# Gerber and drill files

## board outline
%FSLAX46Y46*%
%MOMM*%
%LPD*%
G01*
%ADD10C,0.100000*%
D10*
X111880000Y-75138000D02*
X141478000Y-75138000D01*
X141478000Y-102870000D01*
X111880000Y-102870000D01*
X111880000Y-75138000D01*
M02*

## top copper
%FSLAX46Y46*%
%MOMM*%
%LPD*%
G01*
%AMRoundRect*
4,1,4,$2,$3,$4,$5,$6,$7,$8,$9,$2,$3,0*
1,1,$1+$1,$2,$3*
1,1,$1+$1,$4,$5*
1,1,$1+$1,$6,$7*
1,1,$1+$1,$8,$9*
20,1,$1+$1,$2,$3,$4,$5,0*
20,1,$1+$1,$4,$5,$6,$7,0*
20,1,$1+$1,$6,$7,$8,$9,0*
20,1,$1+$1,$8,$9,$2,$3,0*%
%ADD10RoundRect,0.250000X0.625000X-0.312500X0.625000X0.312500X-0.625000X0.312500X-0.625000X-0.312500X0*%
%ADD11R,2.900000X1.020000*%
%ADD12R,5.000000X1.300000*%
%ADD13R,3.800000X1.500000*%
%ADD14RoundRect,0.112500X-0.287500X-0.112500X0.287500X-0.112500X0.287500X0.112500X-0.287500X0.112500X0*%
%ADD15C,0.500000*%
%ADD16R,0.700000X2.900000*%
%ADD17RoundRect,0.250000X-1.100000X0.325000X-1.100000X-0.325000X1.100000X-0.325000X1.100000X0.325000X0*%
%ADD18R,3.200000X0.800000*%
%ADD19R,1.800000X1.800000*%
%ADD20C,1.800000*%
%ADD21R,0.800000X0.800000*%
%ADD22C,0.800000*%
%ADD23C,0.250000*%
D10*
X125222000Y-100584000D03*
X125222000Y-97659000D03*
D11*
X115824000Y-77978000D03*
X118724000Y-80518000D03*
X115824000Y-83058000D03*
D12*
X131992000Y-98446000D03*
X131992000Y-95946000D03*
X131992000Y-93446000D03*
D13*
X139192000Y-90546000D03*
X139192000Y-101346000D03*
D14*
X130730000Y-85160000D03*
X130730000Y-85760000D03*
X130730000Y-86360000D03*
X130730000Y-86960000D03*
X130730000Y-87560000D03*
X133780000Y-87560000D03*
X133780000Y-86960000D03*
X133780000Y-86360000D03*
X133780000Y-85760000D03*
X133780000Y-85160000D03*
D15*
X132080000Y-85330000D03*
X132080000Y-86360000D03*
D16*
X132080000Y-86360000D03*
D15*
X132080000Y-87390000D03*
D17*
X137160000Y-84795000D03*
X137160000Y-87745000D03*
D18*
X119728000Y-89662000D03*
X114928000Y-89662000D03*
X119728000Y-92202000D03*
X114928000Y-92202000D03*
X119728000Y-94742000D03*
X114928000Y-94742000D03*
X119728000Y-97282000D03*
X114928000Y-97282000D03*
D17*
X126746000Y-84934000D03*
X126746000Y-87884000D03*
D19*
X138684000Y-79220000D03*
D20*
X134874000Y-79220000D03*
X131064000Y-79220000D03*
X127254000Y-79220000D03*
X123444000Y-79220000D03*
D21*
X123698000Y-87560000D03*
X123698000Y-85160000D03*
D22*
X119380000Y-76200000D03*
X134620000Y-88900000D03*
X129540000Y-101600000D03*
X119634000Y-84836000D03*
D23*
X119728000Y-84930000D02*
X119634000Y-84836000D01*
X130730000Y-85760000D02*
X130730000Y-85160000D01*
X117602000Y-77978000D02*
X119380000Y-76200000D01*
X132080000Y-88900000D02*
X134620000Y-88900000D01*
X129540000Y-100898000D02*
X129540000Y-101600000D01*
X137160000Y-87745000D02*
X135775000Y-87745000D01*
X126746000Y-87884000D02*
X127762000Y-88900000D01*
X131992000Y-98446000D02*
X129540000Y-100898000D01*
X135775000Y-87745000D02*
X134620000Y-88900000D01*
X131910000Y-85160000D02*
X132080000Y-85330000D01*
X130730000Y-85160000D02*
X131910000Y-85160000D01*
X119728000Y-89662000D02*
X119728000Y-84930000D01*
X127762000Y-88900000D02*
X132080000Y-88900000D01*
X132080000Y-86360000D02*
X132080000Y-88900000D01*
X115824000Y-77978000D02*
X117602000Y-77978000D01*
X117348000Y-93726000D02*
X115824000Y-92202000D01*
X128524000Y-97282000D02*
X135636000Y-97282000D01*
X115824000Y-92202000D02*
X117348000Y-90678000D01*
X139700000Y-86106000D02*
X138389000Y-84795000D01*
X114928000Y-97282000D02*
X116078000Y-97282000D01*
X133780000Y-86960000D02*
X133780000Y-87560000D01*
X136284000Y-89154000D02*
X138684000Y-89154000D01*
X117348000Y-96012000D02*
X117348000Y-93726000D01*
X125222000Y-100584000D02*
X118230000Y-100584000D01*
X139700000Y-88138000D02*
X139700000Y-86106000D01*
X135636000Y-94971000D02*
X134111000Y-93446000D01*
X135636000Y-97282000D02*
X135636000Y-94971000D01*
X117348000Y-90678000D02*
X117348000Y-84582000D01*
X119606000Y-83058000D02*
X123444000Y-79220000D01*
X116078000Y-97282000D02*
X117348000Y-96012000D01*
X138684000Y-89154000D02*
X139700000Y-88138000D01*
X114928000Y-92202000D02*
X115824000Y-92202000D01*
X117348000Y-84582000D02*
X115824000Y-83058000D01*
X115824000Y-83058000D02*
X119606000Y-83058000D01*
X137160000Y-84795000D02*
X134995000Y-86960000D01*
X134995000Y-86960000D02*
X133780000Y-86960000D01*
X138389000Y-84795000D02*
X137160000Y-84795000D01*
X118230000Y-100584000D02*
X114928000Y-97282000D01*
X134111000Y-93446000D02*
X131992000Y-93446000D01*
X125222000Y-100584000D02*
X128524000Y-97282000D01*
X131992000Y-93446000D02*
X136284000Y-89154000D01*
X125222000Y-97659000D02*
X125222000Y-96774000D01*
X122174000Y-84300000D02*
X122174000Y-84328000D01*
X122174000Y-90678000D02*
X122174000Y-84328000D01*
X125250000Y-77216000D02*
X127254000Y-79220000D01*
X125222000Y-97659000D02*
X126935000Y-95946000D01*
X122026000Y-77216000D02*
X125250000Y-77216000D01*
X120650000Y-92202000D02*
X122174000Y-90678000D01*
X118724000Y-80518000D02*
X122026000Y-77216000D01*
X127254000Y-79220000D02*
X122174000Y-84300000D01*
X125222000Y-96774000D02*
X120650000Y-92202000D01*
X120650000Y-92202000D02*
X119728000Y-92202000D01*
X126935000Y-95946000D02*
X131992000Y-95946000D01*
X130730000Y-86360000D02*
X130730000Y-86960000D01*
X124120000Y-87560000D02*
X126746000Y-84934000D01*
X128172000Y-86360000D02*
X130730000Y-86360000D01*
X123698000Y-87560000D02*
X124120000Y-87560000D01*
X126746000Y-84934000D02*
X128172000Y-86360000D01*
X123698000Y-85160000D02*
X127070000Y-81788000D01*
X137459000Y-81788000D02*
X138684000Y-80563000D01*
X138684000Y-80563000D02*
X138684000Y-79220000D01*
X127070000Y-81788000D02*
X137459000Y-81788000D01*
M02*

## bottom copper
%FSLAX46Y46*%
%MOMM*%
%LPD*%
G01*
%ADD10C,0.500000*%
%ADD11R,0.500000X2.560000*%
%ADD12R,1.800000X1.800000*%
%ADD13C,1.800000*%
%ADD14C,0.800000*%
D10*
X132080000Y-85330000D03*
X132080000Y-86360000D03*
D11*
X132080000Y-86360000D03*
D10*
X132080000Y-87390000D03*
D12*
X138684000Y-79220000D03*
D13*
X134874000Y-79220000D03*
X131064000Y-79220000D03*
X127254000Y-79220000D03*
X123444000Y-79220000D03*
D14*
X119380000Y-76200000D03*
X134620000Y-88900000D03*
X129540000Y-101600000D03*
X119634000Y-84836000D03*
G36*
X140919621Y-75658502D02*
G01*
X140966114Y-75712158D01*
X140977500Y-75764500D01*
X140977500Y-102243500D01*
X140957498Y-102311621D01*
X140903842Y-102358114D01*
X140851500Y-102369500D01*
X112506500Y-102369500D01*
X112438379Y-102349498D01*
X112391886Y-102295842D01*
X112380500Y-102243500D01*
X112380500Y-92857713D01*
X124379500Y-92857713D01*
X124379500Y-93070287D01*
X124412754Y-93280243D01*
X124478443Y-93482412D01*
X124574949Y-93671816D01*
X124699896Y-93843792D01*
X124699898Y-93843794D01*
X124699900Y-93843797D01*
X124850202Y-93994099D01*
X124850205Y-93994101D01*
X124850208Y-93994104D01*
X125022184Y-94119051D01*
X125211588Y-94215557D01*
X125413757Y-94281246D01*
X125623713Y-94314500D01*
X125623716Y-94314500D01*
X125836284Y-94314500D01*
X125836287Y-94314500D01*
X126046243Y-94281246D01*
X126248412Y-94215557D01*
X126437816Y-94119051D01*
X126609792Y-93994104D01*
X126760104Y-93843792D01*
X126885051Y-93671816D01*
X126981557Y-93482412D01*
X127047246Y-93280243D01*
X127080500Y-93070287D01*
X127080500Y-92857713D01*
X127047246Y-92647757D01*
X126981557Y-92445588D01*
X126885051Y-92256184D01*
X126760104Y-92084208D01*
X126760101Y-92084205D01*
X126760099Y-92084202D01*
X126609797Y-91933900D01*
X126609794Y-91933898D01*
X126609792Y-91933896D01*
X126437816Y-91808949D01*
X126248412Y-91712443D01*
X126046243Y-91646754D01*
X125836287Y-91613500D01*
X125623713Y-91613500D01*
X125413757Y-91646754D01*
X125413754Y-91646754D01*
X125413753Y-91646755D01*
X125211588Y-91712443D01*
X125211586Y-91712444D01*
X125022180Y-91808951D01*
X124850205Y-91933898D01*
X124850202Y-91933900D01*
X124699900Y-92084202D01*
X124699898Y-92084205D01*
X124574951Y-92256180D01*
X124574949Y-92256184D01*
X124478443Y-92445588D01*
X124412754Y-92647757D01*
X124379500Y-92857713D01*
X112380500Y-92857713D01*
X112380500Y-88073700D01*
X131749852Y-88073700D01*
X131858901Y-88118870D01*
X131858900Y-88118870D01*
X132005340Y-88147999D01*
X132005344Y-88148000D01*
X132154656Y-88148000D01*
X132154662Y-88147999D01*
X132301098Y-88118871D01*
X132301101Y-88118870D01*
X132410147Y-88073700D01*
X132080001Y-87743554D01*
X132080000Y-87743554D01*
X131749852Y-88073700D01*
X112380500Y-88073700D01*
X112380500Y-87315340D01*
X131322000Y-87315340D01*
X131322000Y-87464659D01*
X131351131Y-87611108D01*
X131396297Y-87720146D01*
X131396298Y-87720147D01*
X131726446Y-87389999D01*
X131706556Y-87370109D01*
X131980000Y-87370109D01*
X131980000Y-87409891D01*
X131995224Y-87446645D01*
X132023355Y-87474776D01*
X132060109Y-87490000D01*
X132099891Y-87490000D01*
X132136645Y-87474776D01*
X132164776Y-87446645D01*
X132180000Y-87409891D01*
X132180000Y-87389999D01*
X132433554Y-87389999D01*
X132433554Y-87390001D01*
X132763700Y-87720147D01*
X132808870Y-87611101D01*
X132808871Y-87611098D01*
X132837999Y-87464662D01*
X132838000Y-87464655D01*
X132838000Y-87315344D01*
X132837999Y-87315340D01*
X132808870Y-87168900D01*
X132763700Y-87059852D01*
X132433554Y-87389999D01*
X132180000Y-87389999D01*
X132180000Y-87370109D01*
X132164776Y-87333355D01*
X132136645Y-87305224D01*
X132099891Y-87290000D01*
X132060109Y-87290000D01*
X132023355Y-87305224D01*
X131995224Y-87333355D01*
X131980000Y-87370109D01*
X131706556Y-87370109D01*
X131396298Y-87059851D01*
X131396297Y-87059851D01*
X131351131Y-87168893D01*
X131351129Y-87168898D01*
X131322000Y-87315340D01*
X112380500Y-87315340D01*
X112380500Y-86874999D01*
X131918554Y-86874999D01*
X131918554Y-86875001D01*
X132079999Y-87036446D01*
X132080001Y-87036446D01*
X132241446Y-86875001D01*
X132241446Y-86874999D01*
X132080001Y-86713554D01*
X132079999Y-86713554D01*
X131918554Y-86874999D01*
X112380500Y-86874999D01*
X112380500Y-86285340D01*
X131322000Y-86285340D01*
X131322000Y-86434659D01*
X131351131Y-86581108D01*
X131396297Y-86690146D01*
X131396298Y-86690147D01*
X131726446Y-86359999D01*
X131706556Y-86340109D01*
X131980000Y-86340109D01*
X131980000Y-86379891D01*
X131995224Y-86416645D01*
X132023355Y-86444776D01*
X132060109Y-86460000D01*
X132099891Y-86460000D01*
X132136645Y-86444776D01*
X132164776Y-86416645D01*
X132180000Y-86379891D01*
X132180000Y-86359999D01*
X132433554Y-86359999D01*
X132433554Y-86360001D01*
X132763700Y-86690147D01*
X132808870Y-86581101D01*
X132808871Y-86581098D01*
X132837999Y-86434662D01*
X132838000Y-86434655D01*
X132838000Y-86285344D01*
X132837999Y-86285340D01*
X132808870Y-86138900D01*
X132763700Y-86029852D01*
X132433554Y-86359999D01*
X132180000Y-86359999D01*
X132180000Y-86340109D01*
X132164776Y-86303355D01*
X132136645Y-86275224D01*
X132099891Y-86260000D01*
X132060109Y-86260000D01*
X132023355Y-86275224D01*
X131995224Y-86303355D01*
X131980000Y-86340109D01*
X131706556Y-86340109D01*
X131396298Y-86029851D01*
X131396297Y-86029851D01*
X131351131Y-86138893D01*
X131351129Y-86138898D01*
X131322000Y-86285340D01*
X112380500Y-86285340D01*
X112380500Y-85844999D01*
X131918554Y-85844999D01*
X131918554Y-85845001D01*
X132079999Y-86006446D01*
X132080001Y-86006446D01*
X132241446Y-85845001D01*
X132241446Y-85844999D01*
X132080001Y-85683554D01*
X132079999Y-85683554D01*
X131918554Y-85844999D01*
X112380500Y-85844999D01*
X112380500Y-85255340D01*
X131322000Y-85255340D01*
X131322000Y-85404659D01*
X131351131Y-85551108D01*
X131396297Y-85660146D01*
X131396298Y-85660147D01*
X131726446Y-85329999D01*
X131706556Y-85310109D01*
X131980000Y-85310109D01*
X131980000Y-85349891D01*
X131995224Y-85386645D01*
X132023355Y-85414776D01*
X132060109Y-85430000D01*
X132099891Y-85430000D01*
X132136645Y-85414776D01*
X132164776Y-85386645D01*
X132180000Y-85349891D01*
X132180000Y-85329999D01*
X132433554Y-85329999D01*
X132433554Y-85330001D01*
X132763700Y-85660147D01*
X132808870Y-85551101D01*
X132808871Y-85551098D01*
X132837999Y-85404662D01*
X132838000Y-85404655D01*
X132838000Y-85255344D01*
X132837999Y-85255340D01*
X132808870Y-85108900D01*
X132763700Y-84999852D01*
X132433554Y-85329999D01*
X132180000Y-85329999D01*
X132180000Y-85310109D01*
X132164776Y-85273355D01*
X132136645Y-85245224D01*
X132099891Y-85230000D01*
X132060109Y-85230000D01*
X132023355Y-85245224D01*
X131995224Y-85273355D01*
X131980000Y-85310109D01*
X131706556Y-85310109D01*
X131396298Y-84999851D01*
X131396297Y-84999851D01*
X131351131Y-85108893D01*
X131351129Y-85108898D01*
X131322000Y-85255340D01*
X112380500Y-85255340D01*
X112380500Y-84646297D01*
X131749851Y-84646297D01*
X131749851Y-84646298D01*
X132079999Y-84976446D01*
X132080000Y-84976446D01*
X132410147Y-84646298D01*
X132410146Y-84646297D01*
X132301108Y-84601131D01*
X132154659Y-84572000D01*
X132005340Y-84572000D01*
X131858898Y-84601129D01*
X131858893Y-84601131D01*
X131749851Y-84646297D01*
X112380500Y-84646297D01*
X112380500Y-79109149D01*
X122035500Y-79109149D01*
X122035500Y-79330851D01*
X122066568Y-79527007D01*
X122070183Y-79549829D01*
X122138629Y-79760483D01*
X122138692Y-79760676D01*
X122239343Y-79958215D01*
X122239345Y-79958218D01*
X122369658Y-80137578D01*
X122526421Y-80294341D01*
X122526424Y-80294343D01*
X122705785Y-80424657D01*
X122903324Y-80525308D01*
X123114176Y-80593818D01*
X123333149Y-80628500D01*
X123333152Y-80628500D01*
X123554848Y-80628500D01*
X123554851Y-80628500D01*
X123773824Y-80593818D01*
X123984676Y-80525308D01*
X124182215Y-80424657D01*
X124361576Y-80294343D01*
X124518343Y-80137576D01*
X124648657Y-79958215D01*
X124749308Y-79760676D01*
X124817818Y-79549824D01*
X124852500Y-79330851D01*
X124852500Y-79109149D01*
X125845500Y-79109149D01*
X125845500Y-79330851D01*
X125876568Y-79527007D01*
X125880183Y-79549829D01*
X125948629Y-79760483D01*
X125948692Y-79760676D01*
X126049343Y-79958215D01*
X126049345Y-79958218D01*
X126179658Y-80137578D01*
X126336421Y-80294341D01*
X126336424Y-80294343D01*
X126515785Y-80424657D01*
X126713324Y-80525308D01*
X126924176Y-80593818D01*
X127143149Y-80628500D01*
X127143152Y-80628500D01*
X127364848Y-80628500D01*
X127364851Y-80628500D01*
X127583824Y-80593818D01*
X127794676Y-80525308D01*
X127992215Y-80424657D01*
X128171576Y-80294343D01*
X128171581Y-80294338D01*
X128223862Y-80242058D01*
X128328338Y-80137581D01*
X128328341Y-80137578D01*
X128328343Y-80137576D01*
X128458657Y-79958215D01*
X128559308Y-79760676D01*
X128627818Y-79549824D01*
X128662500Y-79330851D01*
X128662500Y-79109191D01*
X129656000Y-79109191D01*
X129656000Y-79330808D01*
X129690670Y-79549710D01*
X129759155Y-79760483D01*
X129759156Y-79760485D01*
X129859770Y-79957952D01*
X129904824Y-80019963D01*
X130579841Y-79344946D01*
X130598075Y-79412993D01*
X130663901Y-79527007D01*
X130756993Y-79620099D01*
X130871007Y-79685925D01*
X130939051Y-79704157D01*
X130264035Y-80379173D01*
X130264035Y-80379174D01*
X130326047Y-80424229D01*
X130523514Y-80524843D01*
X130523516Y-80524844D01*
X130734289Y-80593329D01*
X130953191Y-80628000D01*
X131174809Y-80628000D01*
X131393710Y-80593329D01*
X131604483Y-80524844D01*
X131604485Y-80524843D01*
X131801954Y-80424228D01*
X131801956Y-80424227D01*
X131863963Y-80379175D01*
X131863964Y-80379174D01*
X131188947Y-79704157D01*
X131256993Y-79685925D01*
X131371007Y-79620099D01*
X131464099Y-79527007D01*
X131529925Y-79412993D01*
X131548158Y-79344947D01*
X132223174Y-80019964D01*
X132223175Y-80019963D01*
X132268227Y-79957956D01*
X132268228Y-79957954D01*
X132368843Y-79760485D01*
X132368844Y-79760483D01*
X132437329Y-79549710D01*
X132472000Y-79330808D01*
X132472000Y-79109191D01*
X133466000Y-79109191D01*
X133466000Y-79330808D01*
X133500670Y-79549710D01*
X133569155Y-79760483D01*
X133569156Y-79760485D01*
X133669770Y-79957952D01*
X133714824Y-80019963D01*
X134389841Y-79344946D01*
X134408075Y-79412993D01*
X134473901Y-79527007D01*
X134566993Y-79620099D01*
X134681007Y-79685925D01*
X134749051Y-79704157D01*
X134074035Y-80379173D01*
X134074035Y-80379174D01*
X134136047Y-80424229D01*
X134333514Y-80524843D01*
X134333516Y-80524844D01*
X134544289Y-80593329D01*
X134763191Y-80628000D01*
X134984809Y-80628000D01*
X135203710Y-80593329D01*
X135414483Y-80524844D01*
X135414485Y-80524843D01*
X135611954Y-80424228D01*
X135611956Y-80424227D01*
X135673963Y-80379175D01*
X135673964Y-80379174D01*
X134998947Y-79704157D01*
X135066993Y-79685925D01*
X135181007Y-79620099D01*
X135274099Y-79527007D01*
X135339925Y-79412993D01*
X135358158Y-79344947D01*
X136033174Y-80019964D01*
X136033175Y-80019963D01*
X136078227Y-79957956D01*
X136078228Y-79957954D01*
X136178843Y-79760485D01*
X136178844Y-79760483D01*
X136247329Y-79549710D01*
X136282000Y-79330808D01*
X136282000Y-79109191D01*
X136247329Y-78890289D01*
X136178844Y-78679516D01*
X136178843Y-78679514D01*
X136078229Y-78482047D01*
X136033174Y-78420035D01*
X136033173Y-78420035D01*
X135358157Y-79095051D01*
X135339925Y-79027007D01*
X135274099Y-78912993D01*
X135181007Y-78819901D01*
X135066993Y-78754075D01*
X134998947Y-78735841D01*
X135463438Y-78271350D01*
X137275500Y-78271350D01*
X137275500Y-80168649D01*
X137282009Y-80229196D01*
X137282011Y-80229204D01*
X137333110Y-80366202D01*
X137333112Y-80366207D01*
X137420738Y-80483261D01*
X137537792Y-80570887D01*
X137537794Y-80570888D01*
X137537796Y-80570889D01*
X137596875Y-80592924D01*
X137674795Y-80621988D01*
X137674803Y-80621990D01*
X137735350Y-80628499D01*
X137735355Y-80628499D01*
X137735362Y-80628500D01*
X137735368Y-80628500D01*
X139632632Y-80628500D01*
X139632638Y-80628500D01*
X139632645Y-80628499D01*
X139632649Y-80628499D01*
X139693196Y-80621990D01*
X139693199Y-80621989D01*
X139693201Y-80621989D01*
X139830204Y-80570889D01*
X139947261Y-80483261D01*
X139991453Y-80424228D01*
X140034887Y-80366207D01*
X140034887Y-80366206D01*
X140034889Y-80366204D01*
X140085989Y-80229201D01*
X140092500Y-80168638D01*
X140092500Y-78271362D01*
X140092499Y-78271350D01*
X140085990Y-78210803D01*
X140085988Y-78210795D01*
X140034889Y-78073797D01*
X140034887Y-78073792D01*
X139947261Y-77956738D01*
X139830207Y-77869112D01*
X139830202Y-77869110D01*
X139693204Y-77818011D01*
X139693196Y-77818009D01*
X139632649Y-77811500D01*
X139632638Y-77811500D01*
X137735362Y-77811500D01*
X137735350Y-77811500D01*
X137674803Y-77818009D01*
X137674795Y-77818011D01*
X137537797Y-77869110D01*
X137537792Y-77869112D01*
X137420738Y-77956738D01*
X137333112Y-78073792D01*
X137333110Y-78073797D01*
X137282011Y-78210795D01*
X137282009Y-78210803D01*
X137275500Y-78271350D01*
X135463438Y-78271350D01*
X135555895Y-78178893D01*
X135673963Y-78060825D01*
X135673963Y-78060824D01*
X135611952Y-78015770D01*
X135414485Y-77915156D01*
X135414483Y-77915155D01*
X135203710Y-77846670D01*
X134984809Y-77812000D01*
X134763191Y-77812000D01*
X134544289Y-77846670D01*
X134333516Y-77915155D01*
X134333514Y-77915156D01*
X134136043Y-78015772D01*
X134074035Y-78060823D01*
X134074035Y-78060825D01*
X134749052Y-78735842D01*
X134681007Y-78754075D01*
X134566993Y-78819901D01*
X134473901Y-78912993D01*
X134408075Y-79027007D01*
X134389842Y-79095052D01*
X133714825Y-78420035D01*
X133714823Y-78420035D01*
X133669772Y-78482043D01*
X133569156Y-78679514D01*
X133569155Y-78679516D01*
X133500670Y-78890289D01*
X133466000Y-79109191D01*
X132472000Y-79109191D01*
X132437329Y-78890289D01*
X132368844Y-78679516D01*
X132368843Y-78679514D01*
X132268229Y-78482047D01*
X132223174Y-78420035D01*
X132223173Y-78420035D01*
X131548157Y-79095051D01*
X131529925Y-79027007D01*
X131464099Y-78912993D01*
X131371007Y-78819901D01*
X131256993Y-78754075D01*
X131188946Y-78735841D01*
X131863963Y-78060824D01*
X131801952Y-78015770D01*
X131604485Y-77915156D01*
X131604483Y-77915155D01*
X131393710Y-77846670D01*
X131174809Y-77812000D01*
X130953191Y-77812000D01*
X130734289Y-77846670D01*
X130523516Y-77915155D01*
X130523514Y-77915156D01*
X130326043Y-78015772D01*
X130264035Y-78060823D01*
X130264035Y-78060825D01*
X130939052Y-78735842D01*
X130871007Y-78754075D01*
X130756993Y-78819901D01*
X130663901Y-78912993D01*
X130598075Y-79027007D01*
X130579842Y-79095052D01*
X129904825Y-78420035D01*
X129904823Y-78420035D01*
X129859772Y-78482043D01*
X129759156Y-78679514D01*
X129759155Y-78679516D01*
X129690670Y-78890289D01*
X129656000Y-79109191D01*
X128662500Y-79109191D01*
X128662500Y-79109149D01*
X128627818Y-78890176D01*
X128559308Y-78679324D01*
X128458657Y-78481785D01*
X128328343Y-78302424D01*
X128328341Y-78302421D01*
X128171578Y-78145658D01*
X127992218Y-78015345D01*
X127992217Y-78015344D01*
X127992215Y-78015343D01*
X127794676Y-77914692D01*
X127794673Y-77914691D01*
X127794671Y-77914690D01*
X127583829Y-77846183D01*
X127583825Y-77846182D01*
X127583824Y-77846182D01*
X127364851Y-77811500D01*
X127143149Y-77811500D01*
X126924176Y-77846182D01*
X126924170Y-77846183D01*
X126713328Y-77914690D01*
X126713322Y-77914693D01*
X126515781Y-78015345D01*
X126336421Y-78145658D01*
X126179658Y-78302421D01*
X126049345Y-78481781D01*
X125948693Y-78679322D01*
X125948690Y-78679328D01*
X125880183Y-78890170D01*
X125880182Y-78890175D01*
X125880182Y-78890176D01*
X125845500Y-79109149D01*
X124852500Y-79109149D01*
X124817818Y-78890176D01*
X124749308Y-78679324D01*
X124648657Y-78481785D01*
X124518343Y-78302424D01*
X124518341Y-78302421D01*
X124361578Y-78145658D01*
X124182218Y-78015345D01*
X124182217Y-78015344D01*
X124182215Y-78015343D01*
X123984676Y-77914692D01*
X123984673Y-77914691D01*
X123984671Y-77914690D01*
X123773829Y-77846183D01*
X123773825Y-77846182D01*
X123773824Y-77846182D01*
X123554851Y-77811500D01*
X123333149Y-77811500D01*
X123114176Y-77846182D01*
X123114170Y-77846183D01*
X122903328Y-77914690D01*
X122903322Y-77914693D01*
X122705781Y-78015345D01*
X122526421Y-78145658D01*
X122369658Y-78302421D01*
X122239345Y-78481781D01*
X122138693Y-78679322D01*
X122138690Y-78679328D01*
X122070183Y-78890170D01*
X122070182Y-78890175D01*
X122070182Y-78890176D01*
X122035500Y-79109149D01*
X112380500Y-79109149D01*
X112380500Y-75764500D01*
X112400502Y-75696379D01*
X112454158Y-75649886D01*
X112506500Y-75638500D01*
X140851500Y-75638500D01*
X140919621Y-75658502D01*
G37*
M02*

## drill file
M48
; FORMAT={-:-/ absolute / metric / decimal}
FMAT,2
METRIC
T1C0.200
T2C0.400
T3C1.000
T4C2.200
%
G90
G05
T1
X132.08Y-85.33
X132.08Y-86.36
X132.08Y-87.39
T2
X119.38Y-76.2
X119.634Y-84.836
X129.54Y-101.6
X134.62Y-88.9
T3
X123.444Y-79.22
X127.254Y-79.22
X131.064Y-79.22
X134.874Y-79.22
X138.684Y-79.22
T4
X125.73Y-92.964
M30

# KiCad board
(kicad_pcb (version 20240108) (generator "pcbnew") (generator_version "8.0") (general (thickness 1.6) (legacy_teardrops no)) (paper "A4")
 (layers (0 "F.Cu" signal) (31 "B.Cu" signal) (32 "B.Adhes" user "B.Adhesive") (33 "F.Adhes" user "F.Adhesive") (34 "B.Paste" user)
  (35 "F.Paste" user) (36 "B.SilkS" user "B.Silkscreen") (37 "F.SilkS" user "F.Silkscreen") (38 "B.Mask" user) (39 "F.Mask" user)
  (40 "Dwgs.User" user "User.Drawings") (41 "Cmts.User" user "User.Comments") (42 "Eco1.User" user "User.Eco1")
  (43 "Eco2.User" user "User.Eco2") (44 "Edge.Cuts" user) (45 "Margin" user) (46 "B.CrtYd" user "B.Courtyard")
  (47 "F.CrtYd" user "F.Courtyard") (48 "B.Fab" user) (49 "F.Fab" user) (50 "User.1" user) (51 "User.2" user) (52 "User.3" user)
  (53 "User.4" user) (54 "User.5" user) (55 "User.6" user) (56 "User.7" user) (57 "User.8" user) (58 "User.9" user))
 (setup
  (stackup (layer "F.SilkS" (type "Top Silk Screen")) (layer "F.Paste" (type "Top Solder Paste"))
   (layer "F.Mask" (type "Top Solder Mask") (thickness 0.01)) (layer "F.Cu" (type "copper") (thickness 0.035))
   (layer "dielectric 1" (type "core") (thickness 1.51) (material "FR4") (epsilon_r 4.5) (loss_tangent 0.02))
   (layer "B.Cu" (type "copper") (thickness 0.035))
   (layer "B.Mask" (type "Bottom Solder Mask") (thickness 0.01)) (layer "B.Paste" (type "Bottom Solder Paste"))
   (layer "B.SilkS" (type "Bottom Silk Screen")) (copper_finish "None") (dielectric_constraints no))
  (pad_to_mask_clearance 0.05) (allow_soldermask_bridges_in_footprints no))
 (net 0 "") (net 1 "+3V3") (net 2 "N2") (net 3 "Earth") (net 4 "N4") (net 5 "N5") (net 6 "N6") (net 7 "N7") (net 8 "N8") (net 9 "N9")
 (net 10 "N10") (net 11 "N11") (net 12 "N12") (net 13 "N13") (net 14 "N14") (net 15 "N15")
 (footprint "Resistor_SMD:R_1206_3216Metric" (layer "F.Cu") (at 125.222 99.1215 90)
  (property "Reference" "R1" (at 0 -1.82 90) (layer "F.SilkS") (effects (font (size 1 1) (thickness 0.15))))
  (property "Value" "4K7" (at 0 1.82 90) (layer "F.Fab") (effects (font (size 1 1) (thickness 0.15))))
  (pad "1" smd roundrect (at -1.4625 0 90) (size 1.125 1.75) (layers "F.Cu" "F.Paste" "F.Mask") (roundrect_rratio 0.222222) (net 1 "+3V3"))
  (pad "2" smd roundrect (at 1.4625 0 90) (size 1.125 1.75) (layers "F.Cu" "F.Paste" "F.Mask") (roundrect_rratio 0.222222) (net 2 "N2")))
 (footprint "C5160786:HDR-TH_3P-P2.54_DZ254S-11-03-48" (layer "F.Cu") (at 117.274 80.518 -90)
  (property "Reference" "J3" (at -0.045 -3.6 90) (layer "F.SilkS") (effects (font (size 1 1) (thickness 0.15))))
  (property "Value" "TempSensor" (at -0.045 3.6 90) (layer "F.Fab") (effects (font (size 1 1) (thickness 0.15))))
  (pad "1" smd rect (at -2.54 1.45 270) (size 1.02 2.9) (layers "F.Cu" "F.Paste" "F.Mask") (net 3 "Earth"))
  (pad "2" smd rect (at 0 -1.45 270) (size 1.02 2.9) (layers "F.Cu" "F.Paste" "F.Mask") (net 2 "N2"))
  (pad "3" smd rect (at 2.54 1.45 270) (size 1.02 2.9) (layers "F.Cu" "F.Paste" "F.Mask") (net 1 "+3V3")))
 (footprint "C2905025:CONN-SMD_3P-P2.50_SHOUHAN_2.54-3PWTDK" (layer "F.Cu") (at 135.592 95.946 90)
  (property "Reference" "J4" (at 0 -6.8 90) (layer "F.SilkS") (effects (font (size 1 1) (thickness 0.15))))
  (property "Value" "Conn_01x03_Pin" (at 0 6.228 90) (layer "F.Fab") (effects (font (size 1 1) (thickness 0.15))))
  (pad "1" smd rect (at -2.5 -3.6 90) (size 1.3 5) (layers "F.Cu" "F.Paste" "F.Mask") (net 3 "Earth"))
  (pad "2" smd rect (at 0 -3.6 90) (size 1.3 5) (layers "F.Cu" "F.Paste" "F.Mask") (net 2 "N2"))
  (pad "3" smd rect (at 2.5 -3.6 90) (size 1.3 5) (layers "F.Cu" "F.Paste" "F.Mask") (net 1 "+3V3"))
  (pad "4" smd rect (at 5.4 3.6 90) (size 1.5 3.8) (layers "F.Cu" "F.Paste" "F.Mask") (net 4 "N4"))
  (pad "5" smd rect (at -5.4 3.6 90) (size 1.5 3.8) (layers "F.Cu" "F.Paste" "F.Mask") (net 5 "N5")))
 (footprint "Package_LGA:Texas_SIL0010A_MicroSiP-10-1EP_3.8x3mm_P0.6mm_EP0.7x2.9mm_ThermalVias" (layer "F.Cu") (at 132.255 86.36)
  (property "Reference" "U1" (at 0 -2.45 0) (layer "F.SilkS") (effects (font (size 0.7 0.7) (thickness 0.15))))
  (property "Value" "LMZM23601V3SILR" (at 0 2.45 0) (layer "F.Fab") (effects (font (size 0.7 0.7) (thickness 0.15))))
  (pad "" smd roundrect (at -0.175 -0.97) (size 0.65 0.9) (layers "F.Paste") (roundrect_rratio 0.25))
  (pad "" smd roundrect (at -0.175 0) (size 0.65 0.9) (layers "F.Paste") (roundrect_rratio 0.25))
  (pad "" smd roundrect (at -0.175 0.97) (size 0.65 0.9) (layers "F.Paste") (roundrect_rratio 0.25))
  (pad "1" smd roundrect (at -1.525 -1.2) (size 0.8 0.45) (layers "F.Cu" "F.Paste" "F.Mask") (roundrect_rratio 0.25) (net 3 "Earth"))
  (pad "2" smd roundrect (at -1.525 -0.6) (size 0.8 0.45) (layers "F.Cu" "F.Paste" "F.Mask") (roundrect_rratio 0.25) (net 3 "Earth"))
  (pad "3" smd roundrect (at -1.525 0) (size 0.8 0.45) (layers "F.Cu" "F.Paste" "F.Mask") (roundrect_rratio 0.25) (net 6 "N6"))
  (pad "4" smd roundrect (at -1.525 0.6) (size 0.8 0.45) (layers "F.Cu" "F.Paste" "F.Mask") (roundrect_rratio 0.25) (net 6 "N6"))
  (pad "5" smd roundrect (at -1.525 1.2) (size 0.8 0.45) (layers "F.Cu" "F.Paste" "F.Mask") (roundrect_rratio 0.25) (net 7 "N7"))
  (pad "6" smd roundrect (at 1.525 1.2) (size 0.8 0.45) (layers "F.Cu" "F.Paste" "F.Mask") (roundrect_rratio 0.25) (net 1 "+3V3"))
  (pad "7" smd roundrect (at 1.525 0.6) (size 0.8 0.45) (layers "F.Cu" "F.Paste" "F.Mask") (roundrect_rratio 0.25) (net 1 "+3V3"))
  (pad "8" smd roundrect (at 1.525 0) (size 0.8 0.45) (layers "F.Cu" "F.Paste" "F.Mask") (roundrect_rratio 0.25) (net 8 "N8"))
  (pad "9" smd roundrect (at 1.525 -0.6) (size 0.8 0.45) (layers "F.Cu" "F.Paste" "F.Mask") (roundrect_rratio 0.25) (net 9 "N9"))
  (pad "10" smd roundrect (at 1.525 -1.2) (size 0.8 0.45) (layers "F.Cu" "F.Paste" "F.Mask") (roundrect_rratio 0.25) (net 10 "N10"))
  (pad "11" thru_hole circle (at -0.175 -1.03) (size 0.5 0.5) (drill 0.2) (layers "*.Cu") (remove_unused_layers no) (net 3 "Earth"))
  (pad "11" thru_hole circle (at -0.175 0) (size 0.5 0.5) (drill 0.2) (layers "*.Cu") (remove_unused_layers no) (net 3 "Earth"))
  (pad "11" smd rect (at -0.175 0) (size 0.5 2.56) (layers "B.Cu") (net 3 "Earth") (zone_connect 2))
  (pad "11" smd rect (at -0.175 0) (size 0.7 2.9) (layers "F.Cu" "F.Mask") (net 3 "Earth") (zone_connect 2))
  (pad "11" thru_hole circle (at -0.175 1.03) (size 0.5 0.5) (drill 0.2) (layers "*.Cu") (remove_unused_layers no) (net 3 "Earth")))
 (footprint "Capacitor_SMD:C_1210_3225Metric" (layer "F.Cu") (at 137.16 86.27 -90)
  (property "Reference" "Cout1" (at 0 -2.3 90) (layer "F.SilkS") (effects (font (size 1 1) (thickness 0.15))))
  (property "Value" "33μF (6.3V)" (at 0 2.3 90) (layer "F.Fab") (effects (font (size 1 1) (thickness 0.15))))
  (pad "1" smd roundrect (at -1.475 0 270) (size 1.15 2.7) (layers "F.Cu" "F.Paste" "F.Mask") (roundrect_rratio 0.217391) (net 1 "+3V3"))
  (pad "2" smd roundrect (at 1.475 0 270) (size 1.15 2.7) (layers "F.Cu" "F.Paste" "F.Mask") (roundrect_rratio 0.217391) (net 3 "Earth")))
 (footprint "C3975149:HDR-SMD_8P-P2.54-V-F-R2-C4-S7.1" (layer "F.Cu") (at 117.328 93.472 -90)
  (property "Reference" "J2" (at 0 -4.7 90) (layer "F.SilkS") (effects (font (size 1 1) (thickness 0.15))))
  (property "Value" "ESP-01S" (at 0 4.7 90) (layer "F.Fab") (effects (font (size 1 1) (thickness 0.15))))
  (pad "1" smd rect (at -3.81 -2.4 270) (size 0.8 3.2) (layers "F.Cu" "F.Paste" "F.Mask") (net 3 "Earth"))
  (pad "2" smd rect (at -3.81 2.4 270) (size 0.8 3.2) (layers "F.Cu" "F.Paste" "F.Mask") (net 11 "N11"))
  (pad "3" smd rect (at -1.27 -2.4 270) (size 0.8 3.2) (layers "F.Cu" "F.Paste" "F.Mask") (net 2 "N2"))
  (pad "4" smd rect (at -1.27 2.4 270) (size 0.8 3.2) (layers "F.Cu" "F.Paste" "F.Mask") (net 1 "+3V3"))
  (pad "5" smd rect (at 1.27 -2.4 270) (size 0.8 3.2) (layers "F.Cu" "F.Paste" "F.Mask") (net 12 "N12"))
  (pad "6" smd rect (at 1.27 2.4 270) (size 0.8 3.2) (layers "F.Cu" "F.Paste" "F.Mask") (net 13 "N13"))
  (pad "7" smd rect (at 3.81 -2.4 270) (size 0.8 3.2) (layers "F.Cu" "F.Paste" "F.Mask") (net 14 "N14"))
  (pad "8" smd rect (at 3.81 2.4 270) (size 0.8 3.2) (layers "F.Cu" "F.Paste" "F.Mask") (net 1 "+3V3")))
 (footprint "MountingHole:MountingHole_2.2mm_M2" (layer "F.Cu") (at 125.73 92.964)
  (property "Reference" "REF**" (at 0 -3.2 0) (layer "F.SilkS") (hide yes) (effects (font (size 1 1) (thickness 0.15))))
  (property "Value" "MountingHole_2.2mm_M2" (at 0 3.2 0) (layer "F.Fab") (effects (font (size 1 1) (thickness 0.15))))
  (pad "" np_thru_hole circle (at 0 0) (size 2.2 2.2) (drill 2.2) (layers "*.Cu" "*.Mask")))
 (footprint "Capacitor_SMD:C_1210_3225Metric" (layer "F.Cu") (at 126.746 86.409 -90)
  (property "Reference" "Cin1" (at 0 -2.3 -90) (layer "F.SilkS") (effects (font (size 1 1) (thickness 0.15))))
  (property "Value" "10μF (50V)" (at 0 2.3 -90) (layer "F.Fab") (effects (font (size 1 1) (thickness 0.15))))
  (pad "1" smd roundrect (at -1.475 0 270) (size 1.15 2.7) (layers "F.Cu" "F.Paste" "F.Mask") (roundrect_rratio 0.217391) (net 6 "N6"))
  (pad "2" smd roundrect (at 1.475 0 270) (size 1.15 2.7) (layers "F.Cu" "F.Paste" "F.Mask") (roundrect_rratio 0.217391) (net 3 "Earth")))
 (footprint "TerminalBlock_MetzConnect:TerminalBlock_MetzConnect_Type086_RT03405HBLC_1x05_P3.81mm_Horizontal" (layer "F.Cu")
  (at 138.684 79.22 180)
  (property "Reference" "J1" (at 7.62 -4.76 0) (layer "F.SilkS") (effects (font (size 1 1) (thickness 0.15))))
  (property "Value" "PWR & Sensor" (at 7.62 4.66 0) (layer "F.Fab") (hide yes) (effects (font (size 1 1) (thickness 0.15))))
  (pad "1" thru_hole rect (at 0 0 180) (size 1.8 1.8) (drill 1) (layers "*.Cu" "*.Mask") (remove_unused_layers no) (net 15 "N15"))
  (pad "2" thru_hole circle (at 3.81 0 180) (size 1.8 1.8) (drill 1) (layers "*.Cu" "*.Mask") (remove_unused_layers no) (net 3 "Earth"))
  (pad "3" thru_hole circle (at 7.62 0 180) (size 1.8 1.8) (drill 1) (layers "*.Cu" "*.Mask") (remove_unused_layers no) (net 3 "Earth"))
  (pad "4" thru_hole circle (at 11.43 0 180) (size 1.8 1.8) (drill 1) (layers "*.Cu" "*.Mask") (remove_unused_layers no) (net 2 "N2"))
  (pad "5" thru_hole circle (at 15.24 0 180) (size 1.8 1.8) (drill 1) (layers "*.Cu" "*.Mask") (remove_unused_layers no) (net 1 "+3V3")))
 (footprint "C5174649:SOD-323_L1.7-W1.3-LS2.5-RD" (layer "F.Cu") (at 123.698 86.36 90)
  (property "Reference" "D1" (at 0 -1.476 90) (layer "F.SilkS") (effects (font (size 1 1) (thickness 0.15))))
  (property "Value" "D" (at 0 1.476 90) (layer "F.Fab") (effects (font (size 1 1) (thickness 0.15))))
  (pad "1" smd rect (at -1.2 0 90) (size 0.8 0.8) (layers "F.Cu" "F.Paste" "F.Mask") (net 6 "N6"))
  (pad "2" smd rect (at 1.2 0 90) (size 0.8 0.8) (layers "F.Cu" "F.Paste" "F.Mask") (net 15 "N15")))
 (gr_rect (start 111.88 75.138) (end 141.478 102.87) (stroke (width 0.1) (type solid)) (fill none) (layer "Edge.Cuts"))
 (segment (start 119.728 84.93) (end 119.634 84.836) (width 0.25) (layer "F.Cu") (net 3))
 (segment (start 130.73 85.76) (end 130.73 85.16) (width 0.25) (layer "F.Cu") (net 3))
 (segment (start 117.602 77.978) (end 119.38 76.2) (width 0.25) (layer "F.Cu") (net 3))
 (segment (start 132.08 88.9) (end 134.62 88.9) (width 0.25) (layer "F.Cu") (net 3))
 (segment (start 129.54 100.898) (end 129.54 101.6) (width 0.25) (layer "F.Cu") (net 3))
 (segment (start 137.16 87.745) (end 135.775 87.745) (width 0.25) (layer "F.Cu") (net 3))
 (segment (start 126.746 87.884) (end 127.762 88.9) (width 0.25) (layer "F.Cu") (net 3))
 (segment (start 131.992 98.446) (end 129.54 100.898) (width 0.25) (layer "F.Cu") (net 3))
 (segment (start 135.775 87.745) (end 134.62 88.9) (width 0.25) (layer "F.Cu") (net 3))
 (segment (start 131.91 85.16) (end 132.08 85.33) (width 0.25) (layer "F.Cu") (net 3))
 (segment (start 130.73 85.16) (end 131.91 85.16) (width 0.25) (layer "F.Cu") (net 3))
 (segment (start 119.728 89.662) (end 119.728 84.93) (width 0.25) (layer "F.Cu") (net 3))
 (segment (start 127.762 88.9) (end 132.08 88.9) (width 0.25) (layer "F.Cu") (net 3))
 (segment (start 132.08 86.36) (end 132.08 88.9) (width 0.25) (layer "F.Cu") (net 3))
 (segment (start 115.824 77.978) (end 117.602 77.978) (width 0.25) (layer "F.Cu") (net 3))
 (via (at 119.38 76.2) (size 0.8) (drill 0.4) (layers "F.Cu" "B.Cu") (free yes) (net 3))
 (via (at 134.62 88.9) (size 0.8) (drill 0.4) (layers "F.Cu" "B.Cu") (free yes) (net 3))
 (via (at 129.54 101.6) (size 0.8) (drill 0.4) (layers "F.Cu" "B.Cu") (free yes) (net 3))
 (via (at 119.634 84.836) (size 0.8) (drill 0.4) (layers "F.Cu" "B.Cu") (free yes) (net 3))
 (segment (start 117.348 93.726) (end 115.824 92.202) (width 0.25) (layer "F.Cu") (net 1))
 (segment (start 128.524 97.282) (end 135.636 97.282) (width 0.25) (layer "F.Cu") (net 1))
 (segment (start 115.824 92.202) (end 117.348 90.678) (width 0.25) (layer "F.Cu") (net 1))
 (segment (start 139.7 86.106) (end 138.389 84.795) (width 0.25) (layer "F.Cu") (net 1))
 (segment (start 114.928 97.282) (end 116.078 97.282) (width 0.25) (layer "F.Cu") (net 1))
 (segment (start 133.78 86.96) (end 133.78 87.56) (width 0.25) (layer "F.Cu") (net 1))
 (segment (start 136.284 89.154) (end 138.684 89.154) (width 0.25) (layer "F.Cu") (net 1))
 (segment (start 117.348 96.012) (end 117.348 93.726) (width 0.25) (layer "F.Cu") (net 1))
 (segment (start 125.222 100.584) (end 118.23 100.584) (width 0.25) (layer "F.Cu") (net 1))
 (segment (start 139.7 88.138) (end 139.7 86.106) (width 0.25) (layer "F.Cu") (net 1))
 (segment (start 135.636 94.971) (end 134.111 93.446) (width 0.25) (layer "F.Cu") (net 1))
 (segment (start 135.636 97.282) (end 135.636 94.971) (width 0.25) (layer "F.Cu") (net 1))
 (segment (start 117.348 90.678) (end 117.348 84.582) (width 0.25) (layer "F.Cu") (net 1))
 (segment (start 119.606 83.058) (end 123.444 79.22) (width 0.25) (layer "F.Cu") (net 1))
 (segment (start 116.078 97.282) (end 117.348 96.012) (width 0.25) (layer "F.Cu") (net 1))
 (segment (start 138.684 89.154) (end 139.7 88.138) (width 0.25) (layer "F.Cu") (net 1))
 (segment (start 114.928 92.202) (end 115.824 92.202) (width 0.25) (layer "F.Cu") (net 1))
 (segment (start 117.348 84.582) (end 115.824 83.058) (width 0.25) (layer "F.Cu") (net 1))
 (segment (start 115.824 83.058) (end 119.606 83.058) (width 0.25) (layer "F.Cu") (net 1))
 (segment (start 137.16 84.795) (end 134.995 86.96) (width 0.25) (layer "F.Cu") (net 1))
 (segment (start 134.995 86.96) (end 133.78 86.96) (width 0.25) (layer "F.Cu") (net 1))
 (segment (start 138.389 84.795) (end 137.16 84.795) (width 0.25) (layer "F.Cu") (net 1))
 (segment (start 118.23 100.584) (end 114.928 97.282) (width 0.25) (layer "F.Cu") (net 1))
 (segment (start 134.111 93.446) (end 131.992 93.446) (width 0.25) (layer "F.Cu") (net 1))
 (segment (start 125.222 100.584) (end 128.524 97.282) (width 0.25) (layer "F.Cu") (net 1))
 (segment (start 131.992 93.446) (end 136.284 89.154) (width 0.25) (layer "F.Cu") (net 1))
 (segment (start 125.222 97.659) (end 125.222 96.774) (width 0.25) (layer "F.Cu") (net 2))
 (segment (start 122.174 84.3) (end 122.174 84.328) (width 0.25) (layer "F.Cu") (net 2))
 (segment (start 122.174 90.678) (end 122.174 84.328) (width 0.25) (layer "F.Cu") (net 2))
 (segment (start 125.25 77.216) (end 127.254 79.22) (width 0.25) (layer "F.Cu") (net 2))
 (segment (start 125.222 97.659) (end 126.935 95.946) (width 0.25) (layer "F.Cu") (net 2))
 (segment (start 122.026 77.216) (end 125.25 77.216) (width 0.25) (layer "F.Cu") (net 2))
 (segment (start 120.65 92.202) (end 122.174 90.678) (width 0.25) (layer "F.Cu") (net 2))
 (segment (start 118.724 80.518) (end 122.026 77.216) (width 0.25) (layer "F.Cu") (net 2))
 (segment (start 127.254 79.22) (end 122.174 84.3) (width 0.25) (layer "F.Cu") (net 2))
 (segment (start 125.222 96.774) (end 120.65 92.202) (width 0.25) (layer "F.Cu") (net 2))
 (segment (start 120.65 92.202) (end 119.728 92.202) (width 0.25) (layer "F.Cu") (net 2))
 (segment (start 126.935 95.946) (end 131.992 95.946) (width 0.25) (layer "F.Cu") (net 2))
 (segment (start 130.73 86.36) (end 130.73 86.96) (width 0.25) (layer "F.Cu") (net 6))
 (segment (start 124.12 87.56) (end 126.746 84.934) (width 0.25) (layer "F.Cu") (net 6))
 (segment (start 128.172 86.36) (end 130.73 86.36) (width 0.25) (layer "F.Cu") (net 6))
 (segment (start 123.698 87.56) (end 124.12 87.56) (width 0.25) (layer "F.Cu") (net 6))
 (segment (start 126.746 84.934) (end 128.172 86.36) (width 0.25) (layer "F.Cu") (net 6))
 (segment (start 123.698 85.16) (end 127.07 81.788) (width 0.25) (layer "F.Cu") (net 15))
 (segment (start 137.459 81.788) (end 138.684 80.563) (width 0.25) (layer "F.Cu") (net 15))
 (segment (start 138.684 80.563) (end 138.684 79.22) (width 0.25) (layer "F.Cu") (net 15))
 (segment (start 127.07 81.788) (end 137.459 81.788) (width 0.25) (layer "F.Cu") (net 15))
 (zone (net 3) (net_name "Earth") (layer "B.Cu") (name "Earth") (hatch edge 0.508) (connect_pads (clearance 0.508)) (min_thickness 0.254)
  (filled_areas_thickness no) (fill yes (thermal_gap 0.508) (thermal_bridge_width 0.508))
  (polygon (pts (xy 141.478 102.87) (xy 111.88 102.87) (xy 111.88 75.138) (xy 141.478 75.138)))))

